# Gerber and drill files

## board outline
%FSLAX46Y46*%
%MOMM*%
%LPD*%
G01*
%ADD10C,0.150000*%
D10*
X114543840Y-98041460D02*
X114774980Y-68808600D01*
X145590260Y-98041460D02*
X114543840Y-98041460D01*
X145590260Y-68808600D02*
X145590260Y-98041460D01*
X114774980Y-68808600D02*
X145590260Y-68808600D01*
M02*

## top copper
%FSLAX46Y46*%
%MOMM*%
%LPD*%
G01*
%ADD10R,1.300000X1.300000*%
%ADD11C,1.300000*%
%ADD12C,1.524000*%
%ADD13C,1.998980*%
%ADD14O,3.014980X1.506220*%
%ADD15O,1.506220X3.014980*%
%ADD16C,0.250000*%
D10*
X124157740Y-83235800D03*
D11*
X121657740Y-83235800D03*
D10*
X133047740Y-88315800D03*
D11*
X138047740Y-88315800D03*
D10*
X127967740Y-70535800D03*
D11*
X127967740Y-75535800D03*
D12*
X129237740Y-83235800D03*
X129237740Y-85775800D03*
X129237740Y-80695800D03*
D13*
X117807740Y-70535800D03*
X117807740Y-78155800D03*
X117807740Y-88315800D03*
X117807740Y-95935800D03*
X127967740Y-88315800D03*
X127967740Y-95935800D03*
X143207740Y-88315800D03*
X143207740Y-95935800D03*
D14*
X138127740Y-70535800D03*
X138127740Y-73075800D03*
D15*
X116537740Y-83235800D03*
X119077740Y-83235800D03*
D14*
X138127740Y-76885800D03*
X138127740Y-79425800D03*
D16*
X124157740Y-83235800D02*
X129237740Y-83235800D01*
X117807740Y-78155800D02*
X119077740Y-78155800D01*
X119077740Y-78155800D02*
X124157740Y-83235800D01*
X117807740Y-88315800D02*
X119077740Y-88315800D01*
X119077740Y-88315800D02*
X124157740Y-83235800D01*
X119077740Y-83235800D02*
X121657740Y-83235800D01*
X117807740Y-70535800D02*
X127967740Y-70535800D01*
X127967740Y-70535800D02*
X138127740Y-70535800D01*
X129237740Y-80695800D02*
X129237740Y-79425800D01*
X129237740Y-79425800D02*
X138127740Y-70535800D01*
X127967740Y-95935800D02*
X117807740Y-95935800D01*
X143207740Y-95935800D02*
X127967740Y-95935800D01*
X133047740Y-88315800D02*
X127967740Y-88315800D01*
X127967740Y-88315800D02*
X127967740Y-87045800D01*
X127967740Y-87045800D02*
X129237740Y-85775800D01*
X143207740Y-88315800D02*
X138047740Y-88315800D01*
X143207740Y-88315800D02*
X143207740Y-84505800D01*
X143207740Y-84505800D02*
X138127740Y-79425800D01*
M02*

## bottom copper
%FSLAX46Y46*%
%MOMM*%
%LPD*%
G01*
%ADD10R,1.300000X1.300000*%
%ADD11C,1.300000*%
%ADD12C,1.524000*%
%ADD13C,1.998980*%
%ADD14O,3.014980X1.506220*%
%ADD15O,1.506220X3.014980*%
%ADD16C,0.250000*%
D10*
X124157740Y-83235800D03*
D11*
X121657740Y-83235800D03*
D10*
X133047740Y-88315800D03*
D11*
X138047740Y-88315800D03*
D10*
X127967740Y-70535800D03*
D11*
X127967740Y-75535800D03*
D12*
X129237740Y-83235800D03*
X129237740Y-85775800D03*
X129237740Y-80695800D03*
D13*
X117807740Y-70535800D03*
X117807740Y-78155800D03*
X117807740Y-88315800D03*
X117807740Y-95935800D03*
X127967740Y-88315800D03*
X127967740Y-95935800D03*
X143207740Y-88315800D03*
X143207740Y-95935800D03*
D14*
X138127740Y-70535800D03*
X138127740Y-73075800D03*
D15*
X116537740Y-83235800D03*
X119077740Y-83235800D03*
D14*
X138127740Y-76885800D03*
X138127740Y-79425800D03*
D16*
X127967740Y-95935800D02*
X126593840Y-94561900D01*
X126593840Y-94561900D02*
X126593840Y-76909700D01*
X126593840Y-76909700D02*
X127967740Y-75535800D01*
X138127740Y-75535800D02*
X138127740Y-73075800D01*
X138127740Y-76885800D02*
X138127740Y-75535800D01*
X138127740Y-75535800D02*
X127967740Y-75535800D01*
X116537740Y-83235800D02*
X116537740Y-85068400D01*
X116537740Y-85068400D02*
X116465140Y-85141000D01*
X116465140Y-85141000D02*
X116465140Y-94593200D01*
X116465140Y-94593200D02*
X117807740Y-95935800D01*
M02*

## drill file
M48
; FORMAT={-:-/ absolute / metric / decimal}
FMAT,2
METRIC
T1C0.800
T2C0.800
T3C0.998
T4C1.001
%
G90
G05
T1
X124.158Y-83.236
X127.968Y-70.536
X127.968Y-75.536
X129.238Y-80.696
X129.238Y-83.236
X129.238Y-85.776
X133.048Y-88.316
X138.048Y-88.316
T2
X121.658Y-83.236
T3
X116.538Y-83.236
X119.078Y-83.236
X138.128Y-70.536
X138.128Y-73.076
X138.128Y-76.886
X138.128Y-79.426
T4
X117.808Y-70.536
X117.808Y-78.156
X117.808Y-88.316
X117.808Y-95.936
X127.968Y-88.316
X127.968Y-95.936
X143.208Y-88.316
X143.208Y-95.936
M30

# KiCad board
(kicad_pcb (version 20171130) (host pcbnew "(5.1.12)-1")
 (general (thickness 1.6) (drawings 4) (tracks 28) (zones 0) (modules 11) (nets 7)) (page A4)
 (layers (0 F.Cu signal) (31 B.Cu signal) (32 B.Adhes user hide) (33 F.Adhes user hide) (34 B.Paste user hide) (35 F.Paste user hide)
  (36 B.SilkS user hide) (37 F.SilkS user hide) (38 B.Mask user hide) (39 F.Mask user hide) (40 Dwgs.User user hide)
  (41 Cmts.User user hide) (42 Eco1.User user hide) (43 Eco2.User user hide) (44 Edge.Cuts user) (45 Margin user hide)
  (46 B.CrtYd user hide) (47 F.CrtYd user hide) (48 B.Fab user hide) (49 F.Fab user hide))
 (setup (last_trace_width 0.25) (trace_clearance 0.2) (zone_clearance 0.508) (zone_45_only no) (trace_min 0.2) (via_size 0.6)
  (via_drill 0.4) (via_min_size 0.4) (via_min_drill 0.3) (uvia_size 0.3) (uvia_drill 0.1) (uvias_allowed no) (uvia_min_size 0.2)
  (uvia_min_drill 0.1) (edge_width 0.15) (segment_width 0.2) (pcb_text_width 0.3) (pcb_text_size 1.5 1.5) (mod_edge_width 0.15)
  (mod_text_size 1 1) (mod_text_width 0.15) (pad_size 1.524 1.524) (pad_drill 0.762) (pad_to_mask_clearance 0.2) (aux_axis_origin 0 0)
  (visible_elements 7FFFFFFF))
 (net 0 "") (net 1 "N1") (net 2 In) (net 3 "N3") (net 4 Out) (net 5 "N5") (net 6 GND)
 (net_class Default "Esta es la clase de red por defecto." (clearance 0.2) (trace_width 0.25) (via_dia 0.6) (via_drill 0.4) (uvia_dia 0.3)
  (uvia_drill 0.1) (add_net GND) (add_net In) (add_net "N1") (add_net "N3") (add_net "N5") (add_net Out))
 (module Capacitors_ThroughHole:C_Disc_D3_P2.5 (layer F.Cu) (at 124.15774 83.2358 180)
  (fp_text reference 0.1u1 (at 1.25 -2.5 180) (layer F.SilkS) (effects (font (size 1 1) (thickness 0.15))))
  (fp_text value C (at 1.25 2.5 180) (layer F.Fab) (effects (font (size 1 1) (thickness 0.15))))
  (pad 1 thru_hole rect (at 0 0 180) (size 1.3 1.3) (drill 0.8) (layers *.Cu *.Mask) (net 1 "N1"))
  (pad 2 thru_hole circle (at 2.5 0 180) (size 1.3 1.3) (drill 0.8001) (layers *.Cu *.Mask) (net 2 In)))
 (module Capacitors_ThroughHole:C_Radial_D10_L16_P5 (layer F.Cu) (at 133.04774 88.3158)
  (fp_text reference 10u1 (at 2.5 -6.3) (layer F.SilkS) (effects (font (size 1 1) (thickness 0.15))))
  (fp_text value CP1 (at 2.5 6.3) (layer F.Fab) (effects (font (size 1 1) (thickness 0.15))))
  (pad 1 thru_hole rect (at 0 0) (size 1.3 1.3) (drill 0.8) (layers *.Cu *.Mask) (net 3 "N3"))
  (pad 2 thru_hole circle (at 5 0) (size 1.3 1.3) (drill 0.8) (layers *.Cu *.Mask) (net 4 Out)))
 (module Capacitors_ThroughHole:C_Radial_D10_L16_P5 (layer F.Cu) (at 127.96774 70.5358 270)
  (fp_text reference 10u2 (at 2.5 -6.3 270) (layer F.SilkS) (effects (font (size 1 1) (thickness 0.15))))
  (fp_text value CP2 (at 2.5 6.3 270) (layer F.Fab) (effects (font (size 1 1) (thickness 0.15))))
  (pad 1 thru_hole rect (at 0 0 270) (size 1.3 1.3) (drill 0.8) (layers *.Cu *.Mask) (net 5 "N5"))
  (pad 2 thru_hole circle (at 5 0 270) (size 1.3 1.3) (drill 0.8) (layers *.Cu *.Mask) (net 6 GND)))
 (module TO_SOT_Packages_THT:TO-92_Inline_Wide (layer F.Cu) (at 129.23774 80.6958 270)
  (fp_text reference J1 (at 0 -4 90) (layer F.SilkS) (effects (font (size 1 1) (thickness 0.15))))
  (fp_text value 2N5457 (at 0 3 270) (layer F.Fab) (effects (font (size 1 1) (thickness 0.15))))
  (pad 2 thru_hole circle (at 2.54 0) (size 1.524 1.524) (drill 0.8) (layers *.Cu *.Mask) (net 1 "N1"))
  (pad 3 thru_hole circle (at 5.08 0) (size 1.524 1.524) (drill 0.8) (layers *.Cu *.Mask) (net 3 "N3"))
  (pad 1 thru_hole circle (at 0 0) (size 1.524 1.524) (drill 0.8) (layers *.Cu *.Mask) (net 5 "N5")))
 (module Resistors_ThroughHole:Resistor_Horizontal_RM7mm (layer F.Cu) (at 117.80774 70.5358 270)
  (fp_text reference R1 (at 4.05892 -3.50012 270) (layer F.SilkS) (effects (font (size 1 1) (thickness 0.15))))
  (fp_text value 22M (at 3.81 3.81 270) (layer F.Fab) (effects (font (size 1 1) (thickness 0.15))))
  (pad 1 thru_hole circle (at 0 0 270) (size 1.99898 1.99898) (drill 1.00076) (layers *.Cu *.SilkS *.Mask) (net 5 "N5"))
  (pad 2 thru_hole circle (at 7.62 0 270) (size 1.99898 1.99898) (drill 1.00076) (layers *.Cu *.SilkS *.Mask) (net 1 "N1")))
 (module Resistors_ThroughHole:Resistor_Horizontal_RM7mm (layer F.Cu) (at 117.80774 88.3158 270)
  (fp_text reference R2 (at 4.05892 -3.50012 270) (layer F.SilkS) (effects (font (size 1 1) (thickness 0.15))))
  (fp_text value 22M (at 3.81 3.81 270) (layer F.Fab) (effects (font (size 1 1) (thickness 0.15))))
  (pad 1 thru_hole circle (at 0 0 270) (size 1.99898 1.99898) (drill 1.00076) (layers *.Cu *.SilkS *.Mask) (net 1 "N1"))
  (pad 2 thru_hole circle (at 7.62 0 270) (size 1.99898 1.99898) (drill 1.00076) (layers *.Cu *.SilkS *.Mask) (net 6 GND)))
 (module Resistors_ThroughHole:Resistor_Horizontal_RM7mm (layer F.Cu) (at 127.96774 88.3158 270)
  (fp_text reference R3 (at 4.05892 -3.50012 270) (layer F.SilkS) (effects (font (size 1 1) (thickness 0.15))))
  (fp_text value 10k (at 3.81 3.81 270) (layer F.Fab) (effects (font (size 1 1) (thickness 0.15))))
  (pad 1 thru_hole circle (at 0 0 270) (size 1.99898 1.99898) (drill 1.00076) (layers *.Cu *.SilkS *.Mask) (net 3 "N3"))
  (pad 2 thru_hole circle (at 7.62 0 270) (size 1.99898 1.99898) (drill 1.00076) (layers *.Cu *.SilkS *.Mask) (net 6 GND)))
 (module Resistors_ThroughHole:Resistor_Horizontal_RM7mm (layer F.Cu) (at 143.20774 88.3158 270)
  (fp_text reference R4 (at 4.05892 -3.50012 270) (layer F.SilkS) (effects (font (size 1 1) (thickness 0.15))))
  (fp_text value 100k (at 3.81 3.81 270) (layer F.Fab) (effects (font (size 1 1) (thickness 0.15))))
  (pad 1 thru_hole circle (at 0 0 270) (size 1.99898 1.99898) (drill 1.00076) (layers *.Cu *.SilkS *.Mask) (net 4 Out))
  (pad 2 thru_hole circle (at 7.62 0 270) (size 1.99898 1.99898) (drill 1.00076) (layers *.Cu *.SilkS *.Mask) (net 6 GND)))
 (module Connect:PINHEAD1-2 (layer F.Cu) (at 138.12774 71.8058 270)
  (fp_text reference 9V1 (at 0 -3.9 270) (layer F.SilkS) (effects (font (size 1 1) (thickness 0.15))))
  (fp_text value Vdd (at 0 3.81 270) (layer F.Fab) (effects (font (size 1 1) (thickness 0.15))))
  (pad 1 thru_hole oval (at -1.27 0 270) (size 1.50622 3.01498) (drill 0.99822) (layers *.Cu *.Mask) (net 5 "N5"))
  (pad 2 thru_hole oval (at 1.27 0 270) (size 1.50622 3.01498) (drill 0.99822) (layers *.Cu *.Mask) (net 6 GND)))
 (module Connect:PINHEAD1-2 (layer F.Cu) (at 117.80774 83.2358)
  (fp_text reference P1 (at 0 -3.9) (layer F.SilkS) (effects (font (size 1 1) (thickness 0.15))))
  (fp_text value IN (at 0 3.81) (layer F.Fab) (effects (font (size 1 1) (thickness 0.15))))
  (pad 1 thru_hole oval (at -1.27 0) (size 1.50622 3.01498) (drill 0.99822) (layers *.Cu *.Mask) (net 6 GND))
  (pad 2 thru_hole oval (at 1.27 0) (size 1.50622 3.01498) (drill 0.99822) (layers *.Cu *.Mask) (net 2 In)))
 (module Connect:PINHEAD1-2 (layer F.Cu) (at 138.12774 78.1558 270)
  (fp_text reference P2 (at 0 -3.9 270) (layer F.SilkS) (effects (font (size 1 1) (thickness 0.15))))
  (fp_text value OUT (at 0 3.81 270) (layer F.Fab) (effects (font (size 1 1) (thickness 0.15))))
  (pad 1 thru_hole oval (at -1.27 0 270) (size 1.50622 3.01498) (drill 0.99822) (layers *.Cu *.Mask) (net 6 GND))
  (pad 2 thru_hole oval (at 1.27 0 270) (size 1.50622 3.01498) (drill 0.99822) (layers *.Cu *.Mask) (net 4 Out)))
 (gr_line (start 114.54384 98.04146) (end 114.77498 68.8086) (layer Edge.Cuts) (width 0.15))
 (gr_line (start 145.59026 98.04146) (end 114.54384 98.04146) (layer Edge.Cuts) (width 0.15))
 (gr_line (start 145.59026 68.8086) (end 145.59026 98.04146) (layer Edge.Cuts) (width 0.15))
 (gr_line (start 114.77498 68.8086) (end 145.59026 68.8086) (layer Edge.Cuts) (width 0.15))
 (segment (start 124.15774 83.2358) (end 129.23774 83.2358) (width 0.25) (layer F.Cu) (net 1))
 (segment (start 117.80774 78.1558) (end 119.07774 78.1558) (width 0.25) (layer F.Cu) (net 1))
 (segment (start 119.07774 78.1558) (end 124.15774 83.2358) (width 0.25) (layer F.Cu) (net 1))
 (segment (start 117.80774 88.3158) (end 119.07774 88.3158) (width 0.25) (layer F.Cu) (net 1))
 (segment (start 119.07774 88.3158) (end 124.15774 83.2358) (width 0.25) (layer F.Cu) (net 1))
 (segment (start 119.07774 83.2358) (end 121.65774 83.2358) (width 0.25) (layer F.Cu) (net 2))
 (segment (start 117.80774 70.5358) (end 127.96774 70.5358) (width 0.25) (layer F.Cu) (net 5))
 (segment (start 127.96774 70.5358) (end 138.12774 70.5358) (width 0.25) (layer F.Cu) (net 5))
 (segment (start 129.23774 80.6958) (end 129.23774 79.4258) (width 0.25) (layer F.Cu) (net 5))
 (segment (start 129.23774 79.4258) (end 138.12774 70.5358) (width 0.25) (layer F.Cu) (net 5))
 (segment (start 127.96774 95.9358) (end 126.59384 94.5619) (width 0.25) (layer B.Cu) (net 6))
 (segment (start 126.59384 94.5619) (end 126.59384 76.9097) (width 0.25) (layer B.Cu) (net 6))
 (segment (start 126.59384 76.9097) (end 127.96774 75.5358) (width 0.25) (layer B.Cu) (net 6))
 (segment (start 127.96774 95.9358) (end 117.80774 95.9358) (width 0.25) (layer F.Cu) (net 6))
 (segment (start 143.20774 95.9358) (end 127.96774 95.9358) (width 0.25) (layer F.Cu) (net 6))
 (segment (start 138.12774 75.5358) (end 138.12774 73.0758) (width 0.25) (layer B.Cu) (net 6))
 (segment (start 138.12774 76.8858) (end 138.12774 75.5358) (width 0.25) (layer B.Cu) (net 6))
 (segment (start 138.12774 75.5358) (end 127.96774 75.5358) (width 0.25) (layer B.Cu) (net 6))
 (segment (start 116.53774 83.2358) (end 116.53774 85.0684) (width 0.25) (layer B.Cu) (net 6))
 (segment (start 116.53774 85.0684) (end 116.46514 85.141) (width 0.25) (layer B.Cu) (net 6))
 (segment (start 116.46514 85.141) (end 116.46514 94.5932) (width 0.25) (layer B.Cu) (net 6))
 (segment (start 116.46514 94.5932) (end 117.80774 95.9358) (width 0.25) (layer B.Cu) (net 6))
 (segment (start 133.04774 88.3158) (end 127.96774 88.3158) (width 0.25) (layer F.Cu) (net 3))
 (segment (start 127.96774 88.3158) (end 127.96774 87.0458) (width 0.25) (layer F.Cu) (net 3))
 (segment (start 127.96774 87.0458) (end 129.23774 85.7758) (width 0.25) (layer F.Cu) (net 3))
 (segment (start 143.20774 88.3158) (end 138.04774 88.3158) (width 0.25) (layer F.Cu) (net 4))
 (segment (start 143.20774 88.3158) (end 143.20774 84.5058) (width 0.25) (layer F.Cu) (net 4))
 (segment (start 143.20774 84.5058) (end 138.12774 79.4258) (width 0.25) (layer F.Cu) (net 4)))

